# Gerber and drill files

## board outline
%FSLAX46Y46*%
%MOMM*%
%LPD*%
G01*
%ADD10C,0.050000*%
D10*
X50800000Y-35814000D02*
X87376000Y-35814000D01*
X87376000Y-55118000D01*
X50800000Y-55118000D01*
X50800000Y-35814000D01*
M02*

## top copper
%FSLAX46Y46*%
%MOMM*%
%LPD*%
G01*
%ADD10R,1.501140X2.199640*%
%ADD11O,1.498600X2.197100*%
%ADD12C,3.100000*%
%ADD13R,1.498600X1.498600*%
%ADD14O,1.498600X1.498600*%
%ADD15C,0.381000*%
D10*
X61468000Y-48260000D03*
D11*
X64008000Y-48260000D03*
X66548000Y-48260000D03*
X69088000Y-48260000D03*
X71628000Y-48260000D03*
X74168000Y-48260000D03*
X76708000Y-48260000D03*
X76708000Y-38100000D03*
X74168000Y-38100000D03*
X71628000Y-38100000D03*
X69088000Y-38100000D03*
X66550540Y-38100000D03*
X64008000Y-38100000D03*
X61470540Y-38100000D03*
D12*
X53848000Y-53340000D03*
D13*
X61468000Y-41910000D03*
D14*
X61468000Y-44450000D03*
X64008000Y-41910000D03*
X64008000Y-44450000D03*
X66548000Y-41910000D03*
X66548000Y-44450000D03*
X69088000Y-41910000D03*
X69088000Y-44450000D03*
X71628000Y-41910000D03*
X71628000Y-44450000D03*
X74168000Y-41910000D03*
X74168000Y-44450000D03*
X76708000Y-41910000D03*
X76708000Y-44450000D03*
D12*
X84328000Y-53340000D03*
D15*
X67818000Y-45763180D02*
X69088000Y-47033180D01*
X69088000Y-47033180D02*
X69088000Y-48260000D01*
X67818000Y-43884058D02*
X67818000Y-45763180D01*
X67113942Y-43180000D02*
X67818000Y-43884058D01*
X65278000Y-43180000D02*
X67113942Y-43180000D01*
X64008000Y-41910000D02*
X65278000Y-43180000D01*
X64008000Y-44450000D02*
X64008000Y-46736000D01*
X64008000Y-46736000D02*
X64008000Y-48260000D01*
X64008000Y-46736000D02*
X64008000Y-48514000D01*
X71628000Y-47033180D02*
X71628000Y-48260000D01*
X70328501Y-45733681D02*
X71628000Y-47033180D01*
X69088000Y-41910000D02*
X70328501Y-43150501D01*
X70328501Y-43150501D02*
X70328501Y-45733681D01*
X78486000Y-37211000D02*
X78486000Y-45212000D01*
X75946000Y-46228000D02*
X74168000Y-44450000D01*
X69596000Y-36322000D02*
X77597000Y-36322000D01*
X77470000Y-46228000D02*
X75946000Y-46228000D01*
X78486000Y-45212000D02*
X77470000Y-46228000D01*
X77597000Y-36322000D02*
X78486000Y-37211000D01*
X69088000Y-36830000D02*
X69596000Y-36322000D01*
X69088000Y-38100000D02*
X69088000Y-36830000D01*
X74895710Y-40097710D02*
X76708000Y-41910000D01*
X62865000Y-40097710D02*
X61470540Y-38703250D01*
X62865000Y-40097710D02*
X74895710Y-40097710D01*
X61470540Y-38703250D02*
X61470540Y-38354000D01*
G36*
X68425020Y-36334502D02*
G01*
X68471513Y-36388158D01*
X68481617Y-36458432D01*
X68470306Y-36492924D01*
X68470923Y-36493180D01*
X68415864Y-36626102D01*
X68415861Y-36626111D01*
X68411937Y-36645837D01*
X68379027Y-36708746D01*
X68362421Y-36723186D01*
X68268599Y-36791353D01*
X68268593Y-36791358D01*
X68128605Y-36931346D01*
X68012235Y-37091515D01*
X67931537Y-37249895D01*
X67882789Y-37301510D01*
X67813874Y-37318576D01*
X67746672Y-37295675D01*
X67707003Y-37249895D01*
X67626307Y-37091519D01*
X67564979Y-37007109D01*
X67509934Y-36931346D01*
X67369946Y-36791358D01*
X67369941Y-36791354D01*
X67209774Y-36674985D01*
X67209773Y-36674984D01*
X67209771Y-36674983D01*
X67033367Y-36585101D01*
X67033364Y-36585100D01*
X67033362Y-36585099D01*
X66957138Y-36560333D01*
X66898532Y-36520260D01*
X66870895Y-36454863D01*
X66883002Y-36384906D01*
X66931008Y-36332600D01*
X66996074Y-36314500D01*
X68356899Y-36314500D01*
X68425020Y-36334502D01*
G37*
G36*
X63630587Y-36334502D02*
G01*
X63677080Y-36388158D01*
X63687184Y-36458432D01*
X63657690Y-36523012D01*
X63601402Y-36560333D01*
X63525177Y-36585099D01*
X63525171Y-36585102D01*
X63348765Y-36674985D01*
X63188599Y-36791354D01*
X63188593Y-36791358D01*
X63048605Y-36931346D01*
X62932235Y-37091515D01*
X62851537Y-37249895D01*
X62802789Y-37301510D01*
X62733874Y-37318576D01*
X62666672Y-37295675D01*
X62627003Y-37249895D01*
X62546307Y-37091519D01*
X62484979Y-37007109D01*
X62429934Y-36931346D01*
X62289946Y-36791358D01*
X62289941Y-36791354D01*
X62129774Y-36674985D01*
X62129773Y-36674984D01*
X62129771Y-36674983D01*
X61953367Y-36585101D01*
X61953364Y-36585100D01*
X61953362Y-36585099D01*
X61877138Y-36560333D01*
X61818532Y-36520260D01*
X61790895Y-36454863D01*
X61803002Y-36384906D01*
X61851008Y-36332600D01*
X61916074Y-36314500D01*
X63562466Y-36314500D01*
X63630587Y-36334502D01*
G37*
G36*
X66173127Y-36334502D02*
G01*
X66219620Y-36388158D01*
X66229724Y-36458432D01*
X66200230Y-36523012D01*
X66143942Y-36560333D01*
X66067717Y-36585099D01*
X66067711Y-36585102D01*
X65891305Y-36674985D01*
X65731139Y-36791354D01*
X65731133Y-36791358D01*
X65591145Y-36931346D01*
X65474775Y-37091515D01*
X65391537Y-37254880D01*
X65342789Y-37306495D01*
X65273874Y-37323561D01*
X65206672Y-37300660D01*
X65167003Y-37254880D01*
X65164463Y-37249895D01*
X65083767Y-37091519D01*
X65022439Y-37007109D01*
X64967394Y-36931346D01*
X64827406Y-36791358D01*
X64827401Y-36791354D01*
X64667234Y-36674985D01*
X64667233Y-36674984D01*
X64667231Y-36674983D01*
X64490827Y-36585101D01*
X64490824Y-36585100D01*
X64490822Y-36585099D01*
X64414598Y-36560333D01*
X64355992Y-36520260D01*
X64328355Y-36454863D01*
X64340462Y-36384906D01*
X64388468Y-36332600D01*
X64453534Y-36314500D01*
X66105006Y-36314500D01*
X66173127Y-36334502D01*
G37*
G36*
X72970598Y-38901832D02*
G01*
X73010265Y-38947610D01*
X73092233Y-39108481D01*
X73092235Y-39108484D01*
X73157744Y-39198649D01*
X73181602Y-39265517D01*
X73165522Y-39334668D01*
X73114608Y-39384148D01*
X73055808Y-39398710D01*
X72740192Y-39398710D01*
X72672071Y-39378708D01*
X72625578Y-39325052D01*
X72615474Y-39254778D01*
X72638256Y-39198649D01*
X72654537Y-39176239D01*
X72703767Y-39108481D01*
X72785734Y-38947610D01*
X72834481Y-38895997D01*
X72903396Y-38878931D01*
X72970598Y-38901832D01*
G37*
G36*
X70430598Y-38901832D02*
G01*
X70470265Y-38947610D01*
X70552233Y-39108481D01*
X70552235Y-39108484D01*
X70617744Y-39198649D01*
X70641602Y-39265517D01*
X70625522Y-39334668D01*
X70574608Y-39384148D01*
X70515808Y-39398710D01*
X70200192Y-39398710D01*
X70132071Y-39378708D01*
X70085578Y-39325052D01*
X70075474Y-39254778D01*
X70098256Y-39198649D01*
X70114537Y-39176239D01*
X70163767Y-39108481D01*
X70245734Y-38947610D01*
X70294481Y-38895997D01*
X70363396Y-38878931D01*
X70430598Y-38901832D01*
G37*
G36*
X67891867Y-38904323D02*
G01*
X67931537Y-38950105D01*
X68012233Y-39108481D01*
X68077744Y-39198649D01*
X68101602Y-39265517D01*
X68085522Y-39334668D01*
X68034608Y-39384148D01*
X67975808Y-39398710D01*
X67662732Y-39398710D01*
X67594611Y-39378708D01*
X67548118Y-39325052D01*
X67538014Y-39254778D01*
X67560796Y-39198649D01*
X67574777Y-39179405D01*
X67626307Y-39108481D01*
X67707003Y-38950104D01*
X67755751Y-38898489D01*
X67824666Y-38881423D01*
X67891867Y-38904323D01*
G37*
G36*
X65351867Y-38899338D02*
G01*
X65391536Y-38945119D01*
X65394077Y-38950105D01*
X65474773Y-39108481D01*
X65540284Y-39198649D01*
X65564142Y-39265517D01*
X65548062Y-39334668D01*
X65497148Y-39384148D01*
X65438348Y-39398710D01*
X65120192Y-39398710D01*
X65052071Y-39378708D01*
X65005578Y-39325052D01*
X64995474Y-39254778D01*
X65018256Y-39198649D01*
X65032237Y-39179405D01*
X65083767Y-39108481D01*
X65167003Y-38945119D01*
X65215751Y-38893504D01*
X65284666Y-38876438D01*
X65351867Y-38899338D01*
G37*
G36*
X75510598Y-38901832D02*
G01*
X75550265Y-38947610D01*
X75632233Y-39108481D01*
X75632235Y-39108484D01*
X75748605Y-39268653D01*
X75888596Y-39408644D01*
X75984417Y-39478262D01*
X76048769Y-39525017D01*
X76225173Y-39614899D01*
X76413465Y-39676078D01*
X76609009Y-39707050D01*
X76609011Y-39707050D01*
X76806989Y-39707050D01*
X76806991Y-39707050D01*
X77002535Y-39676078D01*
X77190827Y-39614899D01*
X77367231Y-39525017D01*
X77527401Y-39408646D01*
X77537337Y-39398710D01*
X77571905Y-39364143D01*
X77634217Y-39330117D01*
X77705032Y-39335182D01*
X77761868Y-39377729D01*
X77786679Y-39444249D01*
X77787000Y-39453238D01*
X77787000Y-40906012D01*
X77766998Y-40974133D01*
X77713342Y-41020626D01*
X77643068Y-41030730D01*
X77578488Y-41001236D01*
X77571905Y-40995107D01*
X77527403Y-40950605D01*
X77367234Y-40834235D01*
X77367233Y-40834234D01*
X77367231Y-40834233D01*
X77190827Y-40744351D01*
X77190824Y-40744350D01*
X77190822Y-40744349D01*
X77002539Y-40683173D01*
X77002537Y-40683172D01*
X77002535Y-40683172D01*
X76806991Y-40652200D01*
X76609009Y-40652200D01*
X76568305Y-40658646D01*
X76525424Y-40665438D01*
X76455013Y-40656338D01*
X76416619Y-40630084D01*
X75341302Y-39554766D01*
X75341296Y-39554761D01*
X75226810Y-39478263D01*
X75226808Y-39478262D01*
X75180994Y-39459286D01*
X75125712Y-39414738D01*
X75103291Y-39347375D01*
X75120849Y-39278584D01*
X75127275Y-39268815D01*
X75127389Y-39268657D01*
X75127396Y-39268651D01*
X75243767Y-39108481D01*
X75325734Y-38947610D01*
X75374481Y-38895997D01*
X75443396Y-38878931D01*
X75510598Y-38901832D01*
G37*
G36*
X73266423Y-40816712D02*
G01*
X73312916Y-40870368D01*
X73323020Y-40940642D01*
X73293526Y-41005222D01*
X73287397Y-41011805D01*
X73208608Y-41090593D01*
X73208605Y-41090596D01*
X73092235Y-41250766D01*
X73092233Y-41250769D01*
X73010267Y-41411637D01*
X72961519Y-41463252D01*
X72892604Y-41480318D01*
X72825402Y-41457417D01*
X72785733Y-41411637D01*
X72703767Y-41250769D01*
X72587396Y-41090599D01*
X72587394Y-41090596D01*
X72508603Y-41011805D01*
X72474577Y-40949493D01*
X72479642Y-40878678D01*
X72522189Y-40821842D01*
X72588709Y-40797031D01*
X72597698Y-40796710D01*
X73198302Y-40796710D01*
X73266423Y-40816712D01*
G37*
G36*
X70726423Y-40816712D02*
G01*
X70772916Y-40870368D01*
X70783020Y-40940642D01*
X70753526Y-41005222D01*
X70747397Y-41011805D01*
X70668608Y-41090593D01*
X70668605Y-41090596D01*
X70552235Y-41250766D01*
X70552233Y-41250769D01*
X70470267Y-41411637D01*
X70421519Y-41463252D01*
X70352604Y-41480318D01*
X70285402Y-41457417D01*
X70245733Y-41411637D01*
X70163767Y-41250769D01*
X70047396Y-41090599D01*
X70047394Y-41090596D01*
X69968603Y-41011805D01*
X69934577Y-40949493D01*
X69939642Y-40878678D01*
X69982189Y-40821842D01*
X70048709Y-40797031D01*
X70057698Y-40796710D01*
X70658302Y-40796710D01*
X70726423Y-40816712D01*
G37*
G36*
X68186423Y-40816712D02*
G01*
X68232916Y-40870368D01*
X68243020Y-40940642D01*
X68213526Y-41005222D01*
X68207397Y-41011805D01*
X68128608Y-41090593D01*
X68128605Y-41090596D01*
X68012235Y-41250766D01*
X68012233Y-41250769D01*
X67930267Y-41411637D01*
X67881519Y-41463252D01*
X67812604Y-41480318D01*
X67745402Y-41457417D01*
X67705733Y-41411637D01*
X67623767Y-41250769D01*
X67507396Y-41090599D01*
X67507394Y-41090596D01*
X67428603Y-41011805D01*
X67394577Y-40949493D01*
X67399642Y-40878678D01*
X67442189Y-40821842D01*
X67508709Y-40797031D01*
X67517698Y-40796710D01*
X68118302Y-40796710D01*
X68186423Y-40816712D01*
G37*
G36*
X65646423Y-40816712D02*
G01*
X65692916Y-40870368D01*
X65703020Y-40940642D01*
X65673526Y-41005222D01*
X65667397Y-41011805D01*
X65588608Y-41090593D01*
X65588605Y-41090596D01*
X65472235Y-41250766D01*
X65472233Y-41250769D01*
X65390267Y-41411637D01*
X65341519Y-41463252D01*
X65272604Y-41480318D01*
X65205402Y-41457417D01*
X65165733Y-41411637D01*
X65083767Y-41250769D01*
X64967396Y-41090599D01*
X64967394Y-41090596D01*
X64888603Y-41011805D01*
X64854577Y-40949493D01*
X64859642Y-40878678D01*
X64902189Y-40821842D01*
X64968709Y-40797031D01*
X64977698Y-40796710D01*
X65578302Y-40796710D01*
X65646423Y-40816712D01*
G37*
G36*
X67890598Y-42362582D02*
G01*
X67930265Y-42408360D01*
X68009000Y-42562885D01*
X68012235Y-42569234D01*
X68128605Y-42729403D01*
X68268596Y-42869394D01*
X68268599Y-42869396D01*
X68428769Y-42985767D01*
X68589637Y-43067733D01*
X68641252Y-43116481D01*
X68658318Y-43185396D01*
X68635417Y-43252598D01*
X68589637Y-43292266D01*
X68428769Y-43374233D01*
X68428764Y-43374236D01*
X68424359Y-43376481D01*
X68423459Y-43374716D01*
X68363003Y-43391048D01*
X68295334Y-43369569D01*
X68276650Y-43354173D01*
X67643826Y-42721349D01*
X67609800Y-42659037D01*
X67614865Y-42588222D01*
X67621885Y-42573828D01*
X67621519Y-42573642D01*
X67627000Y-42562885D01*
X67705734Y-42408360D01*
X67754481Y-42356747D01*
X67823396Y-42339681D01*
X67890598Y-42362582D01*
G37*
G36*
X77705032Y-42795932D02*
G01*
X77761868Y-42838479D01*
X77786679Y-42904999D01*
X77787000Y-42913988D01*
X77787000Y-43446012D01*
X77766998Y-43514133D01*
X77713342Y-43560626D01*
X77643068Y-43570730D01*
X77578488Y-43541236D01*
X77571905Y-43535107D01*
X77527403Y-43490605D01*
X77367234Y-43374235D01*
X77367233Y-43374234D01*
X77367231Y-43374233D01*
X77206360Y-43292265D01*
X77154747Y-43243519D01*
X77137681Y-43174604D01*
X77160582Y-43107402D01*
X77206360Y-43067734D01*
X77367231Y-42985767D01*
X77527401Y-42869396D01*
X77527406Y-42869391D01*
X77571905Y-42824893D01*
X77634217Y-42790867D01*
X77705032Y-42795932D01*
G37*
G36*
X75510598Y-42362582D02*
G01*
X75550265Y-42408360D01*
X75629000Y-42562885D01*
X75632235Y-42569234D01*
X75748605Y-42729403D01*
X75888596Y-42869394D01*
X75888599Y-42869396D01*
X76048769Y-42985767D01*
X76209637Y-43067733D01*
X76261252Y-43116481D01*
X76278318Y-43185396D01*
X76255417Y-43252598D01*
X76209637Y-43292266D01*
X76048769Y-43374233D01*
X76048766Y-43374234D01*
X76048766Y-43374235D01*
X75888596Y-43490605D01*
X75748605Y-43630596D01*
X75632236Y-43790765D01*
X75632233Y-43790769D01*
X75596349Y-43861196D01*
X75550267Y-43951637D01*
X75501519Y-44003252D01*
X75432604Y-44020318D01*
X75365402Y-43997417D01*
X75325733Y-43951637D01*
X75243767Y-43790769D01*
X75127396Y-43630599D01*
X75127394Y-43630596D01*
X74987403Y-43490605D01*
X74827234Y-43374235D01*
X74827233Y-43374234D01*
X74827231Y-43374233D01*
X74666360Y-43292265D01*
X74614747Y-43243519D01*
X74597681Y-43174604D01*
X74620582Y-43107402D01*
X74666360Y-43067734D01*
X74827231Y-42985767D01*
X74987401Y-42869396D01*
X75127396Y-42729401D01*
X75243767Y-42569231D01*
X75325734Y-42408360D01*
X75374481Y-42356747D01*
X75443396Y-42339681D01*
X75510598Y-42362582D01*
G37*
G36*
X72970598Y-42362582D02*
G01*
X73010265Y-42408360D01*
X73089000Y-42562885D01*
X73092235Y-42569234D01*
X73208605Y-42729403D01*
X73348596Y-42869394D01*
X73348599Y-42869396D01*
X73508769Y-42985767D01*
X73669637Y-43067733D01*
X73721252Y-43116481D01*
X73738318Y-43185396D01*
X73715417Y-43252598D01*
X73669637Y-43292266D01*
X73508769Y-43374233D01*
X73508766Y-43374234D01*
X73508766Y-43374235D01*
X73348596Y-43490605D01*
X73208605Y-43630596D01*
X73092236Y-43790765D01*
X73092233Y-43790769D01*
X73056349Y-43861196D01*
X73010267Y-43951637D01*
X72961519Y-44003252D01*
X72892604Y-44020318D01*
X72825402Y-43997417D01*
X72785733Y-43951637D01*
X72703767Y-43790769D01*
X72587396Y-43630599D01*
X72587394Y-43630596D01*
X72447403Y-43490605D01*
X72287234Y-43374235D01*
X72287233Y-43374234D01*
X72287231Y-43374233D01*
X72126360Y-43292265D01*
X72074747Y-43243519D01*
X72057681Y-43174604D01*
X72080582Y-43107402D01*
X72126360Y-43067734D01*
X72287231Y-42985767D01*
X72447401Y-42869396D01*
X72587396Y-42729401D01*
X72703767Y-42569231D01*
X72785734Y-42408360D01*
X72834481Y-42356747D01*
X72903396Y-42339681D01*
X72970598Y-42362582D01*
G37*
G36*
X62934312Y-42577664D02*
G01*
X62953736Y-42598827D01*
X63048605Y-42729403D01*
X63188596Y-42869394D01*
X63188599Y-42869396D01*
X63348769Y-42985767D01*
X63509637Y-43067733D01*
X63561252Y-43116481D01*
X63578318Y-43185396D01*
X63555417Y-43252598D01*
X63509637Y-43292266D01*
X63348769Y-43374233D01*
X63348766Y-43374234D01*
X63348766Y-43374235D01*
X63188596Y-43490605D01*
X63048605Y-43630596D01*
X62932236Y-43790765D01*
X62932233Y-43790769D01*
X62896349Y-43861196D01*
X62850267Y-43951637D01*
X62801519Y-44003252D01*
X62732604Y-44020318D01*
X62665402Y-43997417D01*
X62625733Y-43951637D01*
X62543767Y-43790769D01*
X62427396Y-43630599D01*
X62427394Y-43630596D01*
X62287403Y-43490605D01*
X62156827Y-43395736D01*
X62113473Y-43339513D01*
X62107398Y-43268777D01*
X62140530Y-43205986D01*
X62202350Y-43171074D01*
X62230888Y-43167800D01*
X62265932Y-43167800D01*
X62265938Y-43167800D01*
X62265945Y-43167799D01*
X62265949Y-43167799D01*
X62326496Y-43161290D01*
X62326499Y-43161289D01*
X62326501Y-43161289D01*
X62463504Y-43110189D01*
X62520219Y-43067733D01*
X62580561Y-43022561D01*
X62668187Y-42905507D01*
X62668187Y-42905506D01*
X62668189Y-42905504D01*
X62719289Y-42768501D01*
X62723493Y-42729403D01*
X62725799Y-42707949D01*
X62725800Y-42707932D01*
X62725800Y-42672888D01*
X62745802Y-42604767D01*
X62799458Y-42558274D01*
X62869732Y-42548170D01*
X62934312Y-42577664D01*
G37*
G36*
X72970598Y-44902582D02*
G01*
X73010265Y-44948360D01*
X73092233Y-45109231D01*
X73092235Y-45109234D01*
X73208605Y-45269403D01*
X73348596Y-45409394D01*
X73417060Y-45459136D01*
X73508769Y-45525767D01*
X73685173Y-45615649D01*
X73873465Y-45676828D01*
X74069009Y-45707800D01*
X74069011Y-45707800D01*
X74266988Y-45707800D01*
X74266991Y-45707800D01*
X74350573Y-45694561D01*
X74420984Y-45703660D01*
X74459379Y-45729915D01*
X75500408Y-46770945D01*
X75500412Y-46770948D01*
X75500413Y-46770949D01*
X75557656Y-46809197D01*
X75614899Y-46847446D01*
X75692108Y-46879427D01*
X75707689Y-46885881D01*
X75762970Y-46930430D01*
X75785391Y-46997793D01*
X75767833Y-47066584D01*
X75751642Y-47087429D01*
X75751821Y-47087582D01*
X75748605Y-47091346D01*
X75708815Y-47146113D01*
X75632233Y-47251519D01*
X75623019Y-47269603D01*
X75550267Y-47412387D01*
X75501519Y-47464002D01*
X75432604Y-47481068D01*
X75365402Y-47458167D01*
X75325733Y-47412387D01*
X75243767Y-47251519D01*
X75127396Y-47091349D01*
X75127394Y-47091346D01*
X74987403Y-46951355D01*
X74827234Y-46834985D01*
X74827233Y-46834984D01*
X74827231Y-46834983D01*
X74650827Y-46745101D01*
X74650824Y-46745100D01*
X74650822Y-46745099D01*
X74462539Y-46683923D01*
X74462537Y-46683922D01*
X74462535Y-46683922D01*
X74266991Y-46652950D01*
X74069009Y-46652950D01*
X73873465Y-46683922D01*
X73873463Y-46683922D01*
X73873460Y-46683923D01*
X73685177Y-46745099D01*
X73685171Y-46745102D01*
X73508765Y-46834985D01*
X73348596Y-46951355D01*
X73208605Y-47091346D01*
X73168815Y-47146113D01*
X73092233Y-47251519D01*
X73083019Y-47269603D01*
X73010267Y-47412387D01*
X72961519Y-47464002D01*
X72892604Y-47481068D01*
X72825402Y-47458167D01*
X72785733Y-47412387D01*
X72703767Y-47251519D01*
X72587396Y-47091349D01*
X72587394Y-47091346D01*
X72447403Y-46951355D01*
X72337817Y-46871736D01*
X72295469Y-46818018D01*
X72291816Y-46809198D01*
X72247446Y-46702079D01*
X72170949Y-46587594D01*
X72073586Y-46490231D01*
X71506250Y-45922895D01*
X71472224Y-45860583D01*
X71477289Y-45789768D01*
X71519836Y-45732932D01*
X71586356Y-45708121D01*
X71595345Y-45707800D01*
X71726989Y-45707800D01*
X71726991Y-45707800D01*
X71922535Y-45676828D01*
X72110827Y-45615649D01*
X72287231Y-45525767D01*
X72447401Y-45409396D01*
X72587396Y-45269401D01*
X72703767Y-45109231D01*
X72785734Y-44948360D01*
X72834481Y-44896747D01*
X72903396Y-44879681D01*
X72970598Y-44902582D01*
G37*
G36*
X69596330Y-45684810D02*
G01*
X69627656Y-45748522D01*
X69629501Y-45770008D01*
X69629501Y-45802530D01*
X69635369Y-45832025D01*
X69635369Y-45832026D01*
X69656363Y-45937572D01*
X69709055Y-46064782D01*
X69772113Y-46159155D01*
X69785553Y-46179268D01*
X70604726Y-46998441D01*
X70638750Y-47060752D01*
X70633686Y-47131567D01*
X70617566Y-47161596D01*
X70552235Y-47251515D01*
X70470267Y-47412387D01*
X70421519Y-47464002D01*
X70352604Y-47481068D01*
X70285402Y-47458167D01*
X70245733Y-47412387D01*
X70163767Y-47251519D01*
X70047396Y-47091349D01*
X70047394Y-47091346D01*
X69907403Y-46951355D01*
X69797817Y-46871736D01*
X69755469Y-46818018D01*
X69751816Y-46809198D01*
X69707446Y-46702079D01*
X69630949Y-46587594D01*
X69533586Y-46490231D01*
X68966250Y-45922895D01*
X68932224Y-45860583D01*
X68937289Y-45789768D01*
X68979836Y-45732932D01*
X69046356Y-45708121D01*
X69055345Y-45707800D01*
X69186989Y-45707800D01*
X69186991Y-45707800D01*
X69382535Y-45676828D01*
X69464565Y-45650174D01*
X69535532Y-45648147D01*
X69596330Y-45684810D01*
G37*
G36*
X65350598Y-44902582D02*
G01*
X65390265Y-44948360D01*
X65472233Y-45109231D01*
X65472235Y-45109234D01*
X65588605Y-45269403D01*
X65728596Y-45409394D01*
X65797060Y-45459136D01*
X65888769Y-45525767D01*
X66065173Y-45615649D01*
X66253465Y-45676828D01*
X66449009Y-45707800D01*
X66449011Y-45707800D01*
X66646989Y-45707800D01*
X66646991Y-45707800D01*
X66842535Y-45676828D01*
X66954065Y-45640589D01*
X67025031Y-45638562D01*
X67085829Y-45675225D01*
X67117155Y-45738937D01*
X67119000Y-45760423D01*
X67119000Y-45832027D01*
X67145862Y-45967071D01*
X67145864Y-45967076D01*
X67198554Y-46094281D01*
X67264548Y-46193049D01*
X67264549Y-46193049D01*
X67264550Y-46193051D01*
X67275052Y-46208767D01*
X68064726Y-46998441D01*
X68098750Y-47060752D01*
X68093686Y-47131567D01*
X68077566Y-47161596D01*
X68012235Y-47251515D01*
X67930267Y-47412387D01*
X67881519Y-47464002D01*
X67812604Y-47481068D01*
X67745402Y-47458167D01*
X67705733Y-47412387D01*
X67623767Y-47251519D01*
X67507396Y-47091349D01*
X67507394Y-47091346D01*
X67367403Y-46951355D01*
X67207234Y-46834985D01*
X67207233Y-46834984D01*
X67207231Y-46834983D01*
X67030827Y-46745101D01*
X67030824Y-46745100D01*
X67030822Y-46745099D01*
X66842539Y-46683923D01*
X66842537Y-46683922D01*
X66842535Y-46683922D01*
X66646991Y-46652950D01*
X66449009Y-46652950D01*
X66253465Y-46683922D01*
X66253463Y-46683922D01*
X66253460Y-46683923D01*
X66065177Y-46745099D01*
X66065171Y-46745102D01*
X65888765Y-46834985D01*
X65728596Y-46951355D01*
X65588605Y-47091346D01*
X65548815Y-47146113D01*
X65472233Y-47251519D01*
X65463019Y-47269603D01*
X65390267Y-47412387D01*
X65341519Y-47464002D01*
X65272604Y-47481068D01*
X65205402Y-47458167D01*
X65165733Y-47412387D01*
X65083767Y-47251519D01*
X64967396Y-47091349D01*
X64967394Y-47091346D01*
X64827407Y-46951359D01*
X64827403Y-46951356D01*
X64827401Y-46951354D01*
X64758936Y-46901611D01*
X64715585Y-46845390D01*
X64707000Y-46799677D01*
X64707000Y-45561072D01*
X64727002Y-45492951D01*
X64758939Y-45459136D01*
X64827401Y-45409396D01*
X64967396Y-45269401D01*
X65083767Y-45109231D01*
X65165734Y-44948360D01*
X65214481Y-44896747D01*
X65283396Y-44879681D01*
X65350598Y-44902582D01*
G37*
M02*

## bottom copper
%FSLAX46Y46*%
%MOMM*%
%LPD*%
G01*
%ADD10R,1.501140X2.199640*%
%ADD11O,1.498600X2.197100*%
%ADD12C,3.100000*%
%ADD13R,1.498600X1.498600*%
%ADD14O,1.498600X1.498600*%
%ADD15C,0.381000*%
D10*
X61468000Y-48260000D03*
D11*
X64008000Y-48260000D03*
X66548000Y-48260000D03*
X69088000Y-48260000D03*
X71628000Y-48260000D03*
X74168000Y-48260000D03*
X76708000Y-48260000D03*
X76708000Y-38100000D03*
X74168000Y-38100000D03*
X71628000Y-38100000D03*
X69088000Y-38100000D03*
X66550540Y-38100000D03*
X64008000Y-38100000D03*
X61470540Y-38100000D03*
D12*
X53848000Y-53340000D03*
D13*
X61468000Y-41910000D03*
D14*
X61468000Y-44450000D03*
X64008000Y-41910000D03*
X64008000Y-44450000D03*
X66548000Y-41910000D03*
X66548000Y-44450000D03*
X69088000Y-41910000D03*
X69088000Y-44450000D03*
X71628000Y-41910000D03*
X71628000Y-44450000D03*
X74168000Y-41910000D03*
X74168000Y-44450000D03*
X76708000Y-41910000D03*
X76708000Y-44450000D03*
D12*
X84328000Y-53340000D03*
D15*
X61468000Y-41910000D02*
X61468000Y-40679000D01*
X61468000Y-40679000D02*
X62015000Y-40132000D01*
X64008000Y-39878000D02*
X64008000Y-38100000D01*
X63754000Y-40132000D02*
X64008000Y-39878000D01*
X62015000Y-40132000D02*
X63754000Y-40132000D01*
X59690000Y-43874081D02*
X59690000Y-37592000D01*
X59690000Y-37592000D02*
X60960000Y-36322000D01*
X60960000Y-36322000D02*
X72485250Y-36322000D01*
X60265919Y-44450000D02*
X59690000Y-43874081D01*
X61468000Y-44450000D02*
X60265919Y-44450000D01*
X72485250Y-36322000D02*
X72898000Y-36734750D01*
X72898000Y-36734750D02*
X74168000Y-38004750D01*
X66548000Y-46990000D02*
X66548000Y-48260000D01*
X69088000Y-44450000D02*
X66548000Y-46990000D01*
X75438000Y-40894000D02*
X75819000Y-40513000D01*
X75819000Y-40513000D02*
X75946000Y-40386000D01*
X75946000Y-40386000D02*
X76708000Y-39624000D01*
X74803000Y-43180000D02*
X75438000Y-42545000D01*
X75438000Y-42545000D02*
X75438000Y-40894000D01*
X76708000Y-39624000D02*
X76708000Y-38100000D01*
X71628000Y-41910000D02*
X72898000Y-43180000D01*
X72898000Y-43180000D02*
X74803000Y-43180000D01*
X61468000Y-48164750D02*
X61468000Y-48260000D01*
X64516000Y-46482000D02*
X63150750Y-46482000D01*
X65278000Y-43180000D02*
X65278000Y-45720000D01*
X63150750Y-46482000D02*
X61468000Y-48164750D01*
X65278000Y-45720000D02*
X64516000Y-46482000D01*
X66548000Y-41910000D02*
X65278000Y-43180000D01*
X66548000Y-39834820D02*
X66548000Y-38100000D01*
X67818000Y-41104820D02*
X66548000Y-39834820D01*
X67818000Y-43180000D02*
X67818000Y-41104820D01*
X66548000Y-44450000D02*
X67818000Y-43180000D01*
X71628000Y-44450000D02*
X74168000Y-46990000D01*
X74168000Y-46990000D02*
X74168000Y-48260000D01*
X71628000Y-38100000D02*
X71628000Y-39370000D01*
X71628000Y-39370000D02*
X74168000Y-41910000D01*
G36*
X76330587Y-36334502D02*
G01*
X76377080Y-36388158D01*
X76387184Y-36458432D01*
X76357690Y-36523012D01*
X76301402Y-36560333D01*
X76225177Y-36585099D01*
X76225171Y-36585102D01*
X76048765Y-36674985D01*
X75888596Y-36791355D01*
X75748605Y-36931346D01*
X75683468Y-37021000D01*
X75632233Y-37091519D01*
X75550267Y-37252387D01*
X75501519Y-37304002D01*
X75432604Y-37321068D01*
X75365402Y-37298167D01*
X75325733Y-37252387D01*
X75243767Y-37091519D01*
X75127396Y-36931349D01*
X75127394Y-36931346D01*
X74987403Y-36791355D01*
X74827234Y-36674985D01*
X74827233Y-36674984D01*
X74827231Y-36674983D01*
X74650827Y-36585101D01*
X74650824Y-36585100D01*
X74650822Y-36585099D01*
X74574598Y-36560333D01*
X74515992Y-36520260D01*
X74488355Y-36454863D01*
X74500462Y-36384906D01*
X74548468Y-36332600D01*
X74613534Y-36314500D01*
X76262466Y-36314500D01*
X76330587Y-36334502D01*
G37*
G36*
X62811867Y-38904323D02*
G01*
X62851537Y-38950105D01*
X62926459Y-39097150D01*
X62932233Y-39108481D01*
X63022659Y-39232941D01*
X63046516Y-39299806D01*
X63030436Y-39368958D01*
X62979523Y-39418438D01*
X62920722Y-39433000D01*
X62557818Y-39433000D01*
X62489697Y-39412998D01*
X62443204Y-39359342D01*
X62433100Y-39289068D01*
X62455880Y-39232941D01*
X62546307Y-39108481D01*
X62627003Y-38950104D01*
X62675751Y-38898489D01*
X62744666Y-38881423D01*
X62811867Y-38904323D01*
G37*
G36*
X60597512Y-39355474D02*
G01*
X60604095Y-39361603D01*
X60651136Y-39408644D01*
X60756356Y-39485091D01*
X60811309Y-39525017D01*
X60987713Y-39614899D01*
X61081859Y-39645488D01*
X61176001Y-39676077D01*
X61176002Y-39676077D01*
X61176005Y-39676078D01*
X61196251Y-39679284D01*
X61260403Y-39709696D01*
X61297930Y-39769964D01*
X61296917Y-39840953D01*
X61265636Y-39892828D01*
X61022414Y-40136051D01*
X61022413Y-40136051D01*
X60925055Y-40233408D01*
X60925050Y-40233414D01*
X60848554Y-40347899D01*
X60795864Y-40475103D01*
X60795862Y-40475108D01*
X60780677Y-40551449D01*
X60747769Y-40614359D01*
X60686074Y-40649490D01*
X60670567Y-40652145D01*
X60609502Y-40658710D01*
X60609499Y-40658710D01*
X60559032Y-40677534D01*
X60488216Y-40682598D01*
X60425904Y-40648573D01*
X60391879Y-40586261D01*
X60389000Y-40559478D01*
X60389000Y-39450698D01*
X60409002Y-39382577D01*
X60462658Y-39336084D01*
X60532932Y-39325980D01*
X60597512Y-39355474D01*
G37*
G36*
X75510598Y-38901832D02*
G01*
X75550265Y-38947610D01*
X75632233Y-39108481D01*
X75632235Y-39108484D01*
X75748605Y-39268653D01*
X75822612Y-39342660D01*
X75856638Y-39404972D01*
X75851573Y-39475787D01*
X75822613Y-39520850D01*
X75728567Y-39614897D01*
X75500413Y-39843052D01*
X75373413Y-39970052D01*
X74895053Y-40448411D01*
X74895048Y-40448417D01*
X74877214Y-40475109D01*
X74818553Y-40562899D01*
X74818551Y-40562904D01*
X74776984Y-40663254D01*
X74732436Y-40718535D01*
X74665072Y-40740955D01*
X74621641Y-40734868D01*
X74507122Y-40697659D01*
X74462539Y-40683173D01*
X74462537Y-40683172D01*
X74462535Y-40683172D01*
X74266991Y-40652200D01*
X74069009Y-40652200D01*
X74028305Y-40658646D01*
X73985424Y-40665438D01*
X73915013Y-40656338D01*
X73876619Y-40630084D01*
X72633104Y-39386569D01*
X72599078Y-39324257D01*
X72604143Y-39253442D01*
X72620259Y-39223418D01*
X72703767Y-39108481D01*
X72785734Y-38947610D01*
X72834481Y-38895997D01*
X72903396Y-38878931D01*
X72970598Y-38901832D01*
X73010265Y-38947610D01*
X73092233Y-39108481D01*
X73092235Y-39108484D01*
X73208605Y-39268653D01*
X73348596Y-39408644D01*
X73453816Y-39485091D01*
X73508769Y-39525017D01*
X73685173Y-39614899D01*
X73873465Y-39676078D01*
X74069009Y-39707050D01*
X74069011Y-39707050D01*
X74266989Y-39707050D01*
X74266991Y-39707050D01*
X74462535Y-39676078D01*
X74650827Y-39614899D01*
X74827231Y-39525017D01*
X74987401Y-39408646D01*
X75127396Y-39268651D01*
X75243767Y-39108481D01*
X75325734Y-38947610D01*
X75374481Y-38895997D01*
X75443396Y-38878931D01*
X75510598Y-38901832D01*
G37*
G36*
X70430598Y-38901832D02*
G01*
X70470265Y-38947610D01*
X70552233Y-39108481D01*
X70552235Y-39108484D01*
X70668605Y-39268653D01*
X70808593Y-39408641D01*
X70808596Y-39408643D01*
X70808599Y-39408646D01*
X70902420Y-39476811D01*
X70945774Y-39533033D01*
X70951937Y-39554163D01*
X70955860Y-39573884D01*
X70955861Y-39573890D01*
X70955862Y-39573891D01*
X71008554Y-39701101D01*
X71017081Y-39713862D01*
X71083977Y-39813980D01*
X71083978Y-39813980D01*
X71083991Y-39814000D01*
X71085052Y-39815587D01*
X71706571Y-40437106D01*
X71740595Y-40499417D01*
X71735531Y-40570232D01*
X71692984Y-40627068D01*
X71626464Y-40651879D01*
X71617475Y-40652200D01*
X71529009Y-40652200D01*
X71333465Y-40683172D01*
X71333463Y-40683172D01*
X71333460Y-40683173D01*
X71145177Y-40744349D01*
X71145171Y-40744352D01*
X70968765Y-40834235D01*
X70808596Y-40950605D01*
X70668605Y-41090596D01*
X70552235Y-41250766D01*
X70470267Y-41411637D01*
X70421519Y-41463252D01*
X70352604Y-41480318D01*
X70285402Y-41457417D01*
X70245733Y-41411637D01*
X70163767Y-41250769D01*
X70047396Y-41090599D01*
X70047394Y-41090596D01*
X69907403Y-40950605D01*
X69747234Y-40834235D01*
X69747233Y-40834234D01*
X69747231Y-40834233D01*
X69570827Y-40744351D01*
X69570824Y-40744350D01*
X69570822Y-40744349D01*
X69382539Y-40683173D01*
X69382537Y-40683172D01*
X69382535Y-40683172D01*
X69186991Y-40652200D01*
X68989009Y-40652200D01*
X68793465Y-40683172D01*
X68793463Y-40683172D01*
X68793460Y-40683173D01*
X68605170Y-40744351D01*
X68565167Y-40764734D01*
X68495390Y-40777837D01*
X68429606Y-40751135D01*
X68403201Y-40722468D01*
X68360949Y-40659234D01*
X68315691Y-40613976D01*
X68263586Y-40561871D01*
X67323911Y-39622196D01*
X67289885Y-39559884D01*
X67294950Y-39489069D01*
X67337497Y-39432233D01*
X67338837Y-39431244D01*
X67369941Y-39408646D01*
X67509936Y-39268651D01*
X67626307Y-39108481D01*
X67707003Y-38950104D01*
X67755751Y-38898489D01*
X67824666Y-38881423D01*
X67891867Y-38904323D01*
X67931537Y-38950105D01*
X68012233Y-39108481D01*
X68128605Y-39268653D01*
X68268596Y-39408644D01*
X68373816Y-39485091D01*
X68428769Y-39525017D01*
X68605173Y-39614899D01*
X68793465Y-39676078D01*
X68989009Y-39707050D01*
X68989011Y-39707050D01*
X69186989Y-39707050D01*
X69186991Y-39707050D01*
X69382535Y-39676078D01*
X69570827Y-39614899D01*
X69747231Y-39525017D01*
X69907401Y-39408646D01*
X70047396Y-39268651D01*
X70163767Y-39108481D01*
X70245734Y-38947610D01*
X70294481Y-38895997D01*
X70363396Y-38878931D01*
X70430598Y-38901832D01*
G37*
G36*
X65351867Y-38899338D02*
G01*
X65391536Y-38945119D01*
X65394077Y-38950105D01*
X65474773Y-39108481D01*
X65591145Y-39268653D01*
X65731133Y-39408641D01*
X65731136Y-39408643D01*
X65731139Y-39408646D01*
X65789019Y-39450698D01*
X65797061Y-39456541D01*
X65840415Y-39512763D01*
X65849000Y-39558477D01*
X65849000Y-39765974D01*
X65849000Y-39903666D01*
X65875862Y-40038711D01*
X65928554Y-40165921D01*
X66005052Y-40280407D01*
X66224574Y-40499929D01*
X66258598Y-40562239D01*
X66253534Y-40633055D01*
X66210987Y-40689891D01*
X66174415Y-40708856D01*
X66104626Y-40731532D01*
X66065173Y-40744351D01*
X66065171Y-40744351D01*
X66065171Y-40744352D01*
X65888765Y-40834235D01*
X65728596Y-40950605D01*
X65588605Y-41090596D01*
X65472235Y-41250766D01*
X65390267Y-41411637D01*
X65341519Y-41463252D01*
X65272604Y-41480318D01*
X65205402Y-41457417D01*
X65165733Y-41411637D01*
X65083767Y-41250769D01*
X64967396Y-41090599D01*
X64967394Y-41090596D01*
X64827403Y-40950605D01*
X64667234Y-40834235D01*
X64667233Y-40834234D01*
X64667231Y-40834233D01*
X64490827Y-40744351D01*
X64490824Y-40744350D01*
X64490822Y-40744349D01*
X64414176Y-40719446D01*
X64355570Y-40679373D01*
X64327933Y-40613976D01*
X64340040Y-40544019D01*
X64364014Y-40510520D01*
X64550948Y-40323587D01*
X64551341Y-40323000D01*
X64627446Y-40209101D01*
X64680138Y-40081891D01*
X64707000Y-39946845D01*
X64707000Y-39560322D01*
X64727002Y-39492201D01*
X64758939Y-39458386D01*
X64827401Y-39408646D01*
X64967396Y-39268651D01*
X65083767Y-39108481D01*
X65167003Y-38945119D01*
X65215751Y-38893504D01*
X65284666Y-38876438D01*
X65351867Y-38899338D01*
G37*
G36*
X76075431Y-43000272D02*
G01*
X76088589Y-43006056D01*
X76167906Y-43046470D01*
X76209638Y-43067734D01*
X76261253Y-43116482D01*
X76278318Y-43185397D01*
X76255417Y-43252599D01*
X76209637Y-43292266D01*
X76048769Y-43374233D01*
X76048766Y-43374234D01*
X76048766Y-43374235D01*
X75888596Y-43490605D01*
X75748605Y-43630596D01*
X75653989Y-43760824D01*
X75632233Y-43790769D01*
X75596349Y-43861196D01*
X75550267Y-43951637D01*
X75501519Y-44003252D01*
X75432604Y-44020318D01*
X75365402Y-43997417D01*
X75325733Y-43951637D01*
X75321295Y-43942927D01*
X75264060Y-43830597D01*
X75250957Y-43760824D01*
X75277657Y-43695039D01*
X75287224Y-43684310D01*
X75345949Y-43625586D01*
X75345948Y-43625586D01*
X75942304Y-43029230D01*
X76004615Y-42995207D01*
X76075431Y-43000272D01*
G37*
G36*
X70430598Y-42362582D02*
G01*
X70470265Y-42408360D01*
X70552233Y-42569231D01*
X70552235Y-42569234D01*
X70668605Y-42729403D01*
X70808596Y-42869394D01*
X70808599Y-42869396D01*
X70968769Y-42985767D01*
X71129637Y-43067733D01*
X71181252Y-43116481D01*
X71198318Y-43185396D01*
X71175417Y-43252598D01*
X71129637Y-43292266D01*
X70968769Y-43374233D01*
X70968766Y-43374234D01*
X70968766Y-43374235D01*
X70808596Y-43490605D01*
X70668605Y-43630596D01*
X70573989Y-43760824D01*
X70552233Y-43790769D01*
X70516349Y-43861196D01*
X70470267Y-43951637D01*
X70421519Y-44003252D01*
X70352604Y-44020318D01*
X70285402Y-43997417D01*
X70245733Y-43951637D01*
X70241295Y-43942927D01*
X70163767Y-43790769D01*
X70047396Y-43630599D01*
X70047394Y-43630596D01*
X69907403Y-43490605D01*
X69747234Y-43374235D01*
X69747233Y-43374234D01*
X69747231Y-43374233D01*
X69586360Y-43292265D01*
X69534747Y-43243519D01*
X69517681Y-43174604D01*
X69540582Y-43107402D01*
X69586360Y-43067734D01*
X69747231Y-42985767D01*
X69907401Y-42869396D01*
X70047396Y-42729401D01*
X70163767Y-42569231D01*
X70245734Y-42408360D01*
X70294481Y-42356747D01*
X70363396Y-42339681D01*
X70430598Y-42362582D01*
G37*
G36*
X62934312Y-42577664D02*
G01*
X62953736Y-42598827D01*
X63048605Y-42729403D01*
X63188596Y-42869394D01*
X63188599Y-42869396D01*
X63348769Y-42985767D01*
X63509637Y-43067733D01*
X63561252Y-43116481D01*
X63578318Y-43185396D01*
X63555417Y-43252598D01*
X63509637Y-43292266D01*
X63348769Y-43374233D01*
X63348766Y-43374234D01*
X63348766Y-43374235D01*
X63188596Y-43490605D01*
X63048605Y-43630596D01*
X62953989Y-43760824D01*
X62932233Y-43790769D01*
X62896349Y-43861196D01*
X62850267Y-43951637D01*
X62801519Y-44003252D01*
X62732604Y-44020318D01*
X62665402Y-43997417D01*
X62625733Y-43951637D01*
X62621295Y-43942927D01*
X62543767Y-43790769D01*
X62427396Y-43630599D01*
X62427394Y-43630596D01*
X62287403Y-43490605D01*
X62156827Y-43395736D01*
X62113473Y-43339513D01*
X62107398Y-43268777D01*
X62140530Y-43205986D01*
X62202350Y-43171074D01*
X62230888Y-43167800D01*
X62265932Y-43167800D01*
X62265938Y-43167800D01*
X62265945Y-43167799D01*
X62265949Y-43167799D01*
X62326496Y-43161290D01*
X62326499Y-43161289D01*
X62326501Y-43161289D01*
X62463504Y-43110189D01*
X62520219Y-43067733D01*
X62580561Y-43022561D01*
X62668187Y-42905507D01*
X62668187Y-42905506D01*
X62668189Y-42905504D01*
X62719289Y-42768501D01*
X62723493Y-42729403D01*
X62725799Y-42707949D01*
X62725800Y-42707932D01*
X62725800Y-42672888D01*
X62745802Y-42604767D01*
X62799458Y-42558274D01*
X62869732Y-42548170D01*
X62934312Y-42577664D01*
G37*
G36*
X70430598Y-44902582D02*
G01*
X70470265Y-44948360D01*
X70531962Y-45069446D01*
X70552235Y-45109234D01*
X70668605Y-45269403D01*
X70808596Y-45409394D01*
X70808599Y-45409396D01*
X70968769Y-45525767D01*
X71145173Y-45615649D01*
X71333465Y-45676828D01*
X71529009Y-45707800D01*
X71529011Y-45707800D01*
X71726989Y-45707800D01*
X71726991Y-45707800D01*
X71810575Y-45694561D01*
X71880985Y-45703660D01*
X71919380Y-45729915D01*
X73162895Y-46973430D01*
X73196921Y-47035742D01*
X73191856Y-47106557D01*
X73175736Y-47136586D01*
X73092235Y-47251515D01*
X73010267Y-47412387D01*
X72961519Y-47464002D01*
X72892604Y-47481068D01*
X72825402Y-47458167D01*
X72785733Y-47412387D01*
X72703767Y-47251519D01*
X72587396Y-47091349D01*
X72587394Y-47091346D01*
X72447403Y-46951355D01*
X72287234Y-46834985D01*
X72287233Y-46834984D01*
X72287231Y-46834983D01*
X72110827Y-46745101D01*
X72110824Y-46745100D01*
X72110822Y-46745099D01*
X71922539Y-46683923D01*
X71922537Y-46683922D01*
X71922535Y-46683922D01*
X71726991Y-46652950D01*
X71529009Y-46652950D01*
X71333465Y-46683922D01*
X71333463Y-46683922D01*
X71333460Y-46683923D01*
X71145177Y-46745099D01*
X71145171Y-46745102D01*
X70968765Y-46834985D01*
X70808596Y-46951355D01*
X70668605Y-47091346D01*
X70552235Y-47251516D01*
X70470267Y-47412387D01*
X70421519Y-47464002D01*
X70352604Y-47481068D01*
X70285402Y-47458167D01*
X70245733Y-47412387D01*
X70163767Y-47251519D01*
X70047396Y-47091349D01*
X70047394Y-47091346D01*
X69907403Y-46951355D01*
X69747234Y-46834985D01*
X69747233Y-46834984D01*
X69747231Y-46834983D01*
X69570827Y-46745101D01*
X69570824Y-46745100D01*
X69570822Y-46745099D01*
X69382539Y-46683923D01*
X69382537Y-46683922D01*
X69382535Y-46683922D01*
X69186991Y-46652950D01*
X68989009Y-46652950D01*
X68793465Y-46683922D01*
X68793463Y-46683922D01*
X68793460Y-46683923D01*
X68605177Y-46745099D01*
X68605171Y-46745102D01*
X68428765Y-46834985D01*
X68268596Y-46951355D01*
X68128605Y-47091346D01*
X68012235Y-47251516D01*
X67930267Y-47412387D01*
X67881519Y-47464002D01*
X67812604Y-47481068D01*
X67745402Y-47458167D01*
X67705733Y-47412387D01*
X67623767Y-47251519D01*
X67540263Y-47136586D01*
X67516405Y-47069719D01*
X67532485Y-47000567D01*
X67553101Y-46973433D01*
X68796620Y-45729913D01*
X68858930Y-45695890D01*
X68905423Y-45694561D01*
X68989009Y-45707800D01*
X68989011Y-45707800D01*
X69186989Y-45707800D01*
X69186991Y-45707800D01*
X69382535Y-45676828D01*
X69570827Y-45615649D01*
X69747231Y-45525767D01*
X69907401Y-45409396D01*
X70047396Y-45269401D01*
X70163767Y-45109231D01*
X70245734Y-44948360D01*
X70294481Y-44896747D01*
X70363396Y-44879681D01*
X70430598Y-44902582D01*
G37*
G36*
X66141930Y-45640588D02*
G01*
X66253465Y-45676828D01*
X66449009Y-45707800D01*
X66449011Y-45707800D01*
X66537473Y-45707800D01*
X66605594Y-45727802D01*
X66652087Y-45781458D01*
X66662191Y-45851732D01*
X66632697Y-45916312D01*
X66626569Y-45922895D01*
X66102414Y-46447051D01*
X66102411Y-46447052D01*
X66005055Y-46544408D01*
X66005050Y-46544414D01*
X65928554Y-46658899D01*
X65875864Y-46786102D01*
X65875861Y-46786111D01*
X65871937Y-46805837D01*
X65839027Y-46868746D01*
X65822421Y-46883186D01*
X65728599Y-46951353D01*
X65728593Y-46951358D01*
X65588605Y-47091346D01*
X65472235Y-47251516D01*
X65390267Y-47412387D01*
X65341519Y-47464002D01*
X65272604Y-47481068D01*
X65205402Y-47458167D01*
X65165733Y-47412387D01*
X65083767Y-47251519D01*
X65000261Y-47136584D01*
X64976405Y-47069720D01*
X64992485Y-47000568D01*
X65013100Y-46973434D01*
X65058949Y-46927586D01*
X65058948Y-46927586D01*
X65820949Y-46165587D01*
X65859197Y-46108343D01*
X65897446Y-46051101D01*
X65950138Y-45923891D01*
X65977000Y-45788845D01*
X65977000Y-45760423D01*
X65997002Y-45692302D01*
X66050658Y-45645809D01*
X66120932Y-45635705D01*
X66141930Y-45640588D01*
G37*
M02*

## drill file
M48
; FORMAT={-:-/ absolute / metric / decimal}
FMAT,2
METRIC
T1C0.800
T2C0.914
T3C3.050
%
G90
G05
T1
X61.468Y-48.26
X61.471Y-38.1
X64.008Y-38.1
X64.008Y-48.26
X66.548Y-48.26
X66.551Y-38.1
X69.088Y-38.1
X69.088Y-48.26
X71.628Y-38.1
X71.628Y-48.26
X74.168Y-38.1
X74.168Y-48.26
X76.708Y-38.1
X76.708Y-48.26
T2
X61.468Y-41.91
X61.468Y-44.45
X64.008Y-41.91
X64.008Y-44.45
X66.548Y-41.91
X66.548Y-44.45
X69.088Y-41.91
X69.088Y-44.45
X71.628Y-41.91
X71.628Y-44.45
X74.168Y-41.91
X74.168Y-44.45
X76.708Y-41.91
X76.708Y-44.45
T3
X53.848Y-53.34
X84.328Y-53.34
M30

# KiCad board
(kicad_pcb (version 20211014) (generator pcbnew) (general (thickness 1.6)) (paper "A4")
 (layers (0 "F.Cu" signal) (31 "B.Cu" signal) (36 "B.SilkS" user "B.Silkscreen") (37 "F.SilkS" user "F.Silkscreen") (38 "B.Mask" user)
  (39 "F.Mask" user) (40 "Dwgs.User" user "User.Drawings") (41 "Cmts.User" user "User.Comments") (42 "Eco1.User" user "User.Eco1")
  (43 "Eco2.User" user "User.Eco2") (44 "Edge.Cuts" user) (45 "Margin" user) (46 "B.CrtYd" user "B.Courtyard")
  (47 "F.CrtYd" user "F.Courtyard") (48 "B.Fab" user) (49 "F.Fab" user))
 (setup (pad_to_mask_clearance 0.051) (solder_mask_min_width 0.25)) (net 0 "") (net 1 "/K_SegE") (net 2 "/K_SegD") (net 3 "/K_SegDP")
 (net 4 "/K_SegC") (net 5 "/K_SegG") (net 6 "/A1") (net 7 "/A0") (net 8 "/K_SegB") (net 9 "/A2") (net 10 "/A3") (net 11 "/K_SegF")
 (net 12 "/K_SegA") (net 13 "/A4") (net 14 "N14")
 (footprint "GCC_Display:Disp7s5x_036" (layer "F.Cu") (at 69.088 43.18)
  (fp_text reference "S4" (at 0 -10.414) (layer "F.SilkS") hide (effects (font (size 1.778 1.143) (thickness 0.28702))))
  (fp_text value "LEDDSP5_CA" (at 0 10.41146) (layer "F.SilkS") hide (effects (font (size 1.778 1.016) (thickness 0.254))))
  (pad "1" thru_hole rect locked (at -7.62 5.08 90) (size 2.19964 1.50114) (drill 0.8001) (layers *.Cu *.Mask) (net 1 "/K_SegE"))
  (pad "2" thru_hole oval locked (at -5.08 5.08 90) (size 2.1971 1.4986) (drill 0.8001) (layers *.Cu *.Mask) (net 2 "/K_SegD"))
  (pad "3" thru_hole oval locked (at -2.54 5.08 90) (size 2.1971 1.4986) (drill 0.8001) (layers *.Cu *.Mask) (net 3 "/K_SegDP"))
  (pad "4" thru_hole oval locked (at 0 5.08 90) (size 2.1971 1.4986) (drill 0.8001) (layers *.Cu *.Mask) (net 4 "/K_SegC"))
  (pad "5" thru_hole oval locked (at 2.54 5.08 90) (size 2.1971 1.4986) (drill 0.8001) (layers *.Cu *.Mask) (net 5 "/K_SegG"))
  (pad "6" thru_hole oval locked (at 5.08 5.08 90) (size 2.1971 1.4986) (drill 0.8001) (layers *.Cu *.Mask) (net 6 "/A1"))
  (pad "7" thru_hole oval locked (at 7.62 5.08 90) (size 2.1971 1.4986) (drill 0.8001) (layers *.Cu *.Mask))
  (pad "8" thru_hole oval locked (at 7.62 -5.08 90) (size 2.1971 1.4986) (drill 0.8001) (layers *.Cu *.Mask) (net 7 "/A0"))
  (pad "9" thru_hole oval locked (at 5.08 -5.08 90) (size 2.1971 1.4986) (drill 0.8001) (layers *.Cu *.Mask) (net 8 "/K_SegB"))
  (pad "10" thru_hole oval locked (at 2.54 -5.08 90) (size 2.1971 1.4986) (drill 0.8001) (layers *.Cu *.Mask) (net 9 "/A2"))
  (pad "11" thru_hole oval locked (at 0 -5.08 90) (size 2.1971 1.4986) (drill 0.8001) (layers *.Cu *.Mask) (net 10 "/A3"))
  (pad "12" thru_hole oval locked (at -2.53746 -5.08 90) (size 2.1971 1.4986) (drill 0.8001) (layers *.Cu *.Mask) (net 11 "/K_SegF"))
  (pad "13" thru_hole oval locked (at -5.08 -5.08 90) (size 2.1971 1.4986) (drill 0.8001) (layers *.Cu *.Mask) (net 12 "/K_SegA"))
  (pad "14" thru_hole oval locked (at -7.61746 -5.08 90) (size 2.1971 1.4986) (drill 0.8001) (layers *.Cu *.Mask) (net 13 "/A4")))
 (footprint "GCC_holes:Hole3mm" (layer "B.Cu") (at 53.848 53.34)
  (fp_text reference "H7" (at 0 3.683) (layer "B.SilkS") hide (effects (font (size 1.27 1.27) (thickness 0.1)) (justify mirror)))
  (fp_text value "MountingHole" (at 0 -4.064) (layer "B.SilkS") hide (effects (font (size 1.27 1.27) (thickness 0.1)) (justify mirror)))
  (pad "1" thru_hole circle locked (at 0 0) (size 3.1 3.1) (drill 3.05) (layers *.Cu *.Mask)))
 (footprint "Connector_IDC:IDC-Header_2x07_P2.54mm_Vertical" (layer "B.Cu") (at 61.468 41.91 -90)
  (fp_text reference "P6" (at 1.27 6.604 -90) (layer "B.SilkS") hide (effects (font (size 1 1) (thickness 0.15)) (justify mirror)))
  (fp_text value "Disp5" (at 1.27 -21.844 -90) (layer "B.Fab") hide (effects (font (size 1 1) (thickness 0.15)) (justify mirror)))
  (pad "1" thru_hole rect locked (at 0 0 270) (size 1.4986 1.4986) (drill 0.9144) (layers *.Cu *.Mask) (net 12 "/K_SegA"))
  (pad "2" thru_hole oval locked (at 2.54 0 270) (size 1.4986 1.4986) (drill 0.9144) (layers *.Cu *.Mask) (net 8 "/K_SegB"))
  (pad "3" thru_hole oval locked (at 0 -2.54 270) (size 1.4986 1.4986) (drill 0.9144) (layers *.Cu *.Mask) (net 4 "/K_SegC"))
  (pad "4" thru_hole oval locked (at 2.54 -2.54 270) (size 1.4986 1.4986) (drill 0.9144) (layers *.Cu *.Mask) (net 2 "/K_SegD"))
  (pad "5" thru_hole oval locked (at 0 -5.08 270) (size 1.4986 1.4986) (drill 0.9144) (layers *.Cu *.Mask) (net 1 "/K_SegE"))
  (pad "6" thru_hole oval locked (at 2.54 -5.08 270) (size 1.4986 1.4986) (drill 0.9144) (layers *.Cu *.Mask) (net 11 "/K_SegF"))
  (pad "7" thru_hole oval locked (at 0 -7.62 270) (size 1.4986 1.4986) (drill 0.9144) (layers *.Cu *.Mask) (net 5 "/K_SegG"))
  (pad "8" thru_hole oval locked (at 2.54 -7.62 270) (size 1.4986 1.4986) (drill 0.9144) (layers *.Cu *.Mask) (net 3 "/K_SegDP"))
  (pad "9" thru_hole oval locked (at 0 -10.16 270) (size 1.4986 1.4986) (drill 0.9144) (layers *.Cu *.Mask) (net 7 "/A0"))
  (pad "10" thru_hole oval locked (at 2.54 -10.16 270) (size 1.4986 1.4986) (drill 0.9144) (layers *.Cu *.Mask) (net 6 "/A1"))
  (pad "11" thru_hole oval locked (at 0 -12.7 270) (size 1.4986 1.4986) (drill 0.9144) (layers *.Cu *.Mask) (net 9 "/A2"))
  (pad "12" thru_hole oval locked (at 2.54 -12.7 270) (size 1.4986 1.4986) (drill 0.9144) (layers *.Cu *.Mask) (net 10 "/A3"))
  (pad "13" thru_hole oval locked (at 0 -15.24 270) (size 1.4986 1.4986) (drill 0.9144) (layers *.Cu *.Mask) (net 13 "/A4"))
  (pad "14" thru_hole oval locked (at 2.54 -15.24 270) (size 1.4986 1.4986) (drill 0.9144) (layers *.Cu *.Mask) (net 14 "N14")))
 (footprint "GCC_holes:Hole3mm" (layer "B.Cu") (at 84.328 53.34)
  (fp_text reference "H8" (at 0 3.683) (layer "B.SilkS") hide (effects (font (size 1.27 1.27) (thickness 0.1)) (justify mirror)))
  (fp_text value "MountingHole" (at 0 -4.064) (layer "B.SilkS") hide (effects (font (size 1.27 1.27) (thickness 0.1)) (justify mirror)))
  (pad "1" thru_hole circle locked (at 0 0) (size 3.1 3.1) (drill 3.05) (layers *.Cu *.Mask)))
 (gr_rect (start 50.8 35.814) (end 87.376 55.118) (layer "Edge.Cuts") (width 0.05) (fill none))
 (segment (start 61.468 41.91) (end 61.468 40.679) (width 0.381) (layer "B.Cu") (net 12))
 (segment (start 61.468 40.679) (end 62.015 40.132) (width 0.381) (layer "B.Cu") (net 12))
 (segment (start 64.008 39.878) (end 64.008 38.1) (width 0.381) (layer "B.Cu") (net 12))
 (segment (start 63.754 40.132) (end 64.008 39.878) (width 0.381) (layer "B.Cu") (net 12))
 (segment (start 62.015 40.132) (end 63.754 40.132) (width 0.381) (layer "B.Cu") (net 12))
 (segment (start 59.69 43.874081) (end 59.69 37.592) (width 0.381) (layer "B.Cu") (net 8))
 (segment (start 59.69 37.592) (end 60.96 36.322) (width 0.381) (layer "B.Cu") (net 8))
 (segment (start 60.96 36.322) (end 72.48525 36.322) (width 0.381) (layer "B.Cu") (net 8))
 (segment (start 60.265919 44.45) (end 59.69 43.874081) (width 0.381) (layer "B.Cu") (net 8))
 (segment (start 61.468 44.45) (end 60.265919 44.45) (width 0.381) (layer "B.Cu") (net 8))
 (segment (start 72.48525 36.322) (end 72.898 36.73475) (width 0.381) (layer "B.Cu") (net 8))
 (segment (start 72.898 36.73475) (end 74.168 38.00475) (width 0.381) (layer "B.Cu") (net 8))
 (segment (start 67.818 45.76318) (end 69.088 47.03318) (width 0.381) (layer "F.Cu") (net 4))
 (segment (start 69.088 47.03318) (end 69.088 48.26) (width 0.381) (layer "F.Cu") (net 4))
 (segment (start 67.818 43.884058) (end 67.818 45.76318) (width 0.381) (layer "F.Cu") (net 4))
 (segment (start 67.113942 43.18) (end 67.818 43.884058) (width 0.381) (layer "F.Cu") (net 4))
 (segment (start 65.278 43.18) (end 67.113942 43.18) (width 0.381) (layer "F.Cu") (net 4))
 (segment (start 64.008 41.91) (end 65.278 43.18) (width 0.381) (layer "F.Cu") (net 4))
 (segment (start 66.548 46.99) (end 66.548 48.26) (width 0.381) (layer "B.Cu") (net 3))
 (segment (start 69.088 44.45) (end 66.548 46.99) (width 0.381) (layer "B.Cu") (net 3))
 (segment (start 75.438 40.894) (end 75.819 40.513) (width 0.381) (layer "B.Cu") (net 7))
 (segment (start 75.819 40.513) (end 75.946 40.386) (width 0.381) (layer "B.Cu") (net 7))
 (segment (start 75.946 40.386) (end 76.708 39.624) (width 0.381) (layer "B.Cu") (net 7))
 (segment (start 74.803 43.18) (end 75.438 42.545) (width 0.381) (layer "B.Cu") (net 7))
 (segment (start 75.438 42.545) (end 75.438 40.894) (width 0.381) (layer "B.Cu") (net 7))
 (segment (start 76.708 39.624) (end 76.708 38.1) (width 0.381) (layer "B.Cu") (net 7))
 (segment (start 71.628 41.91) (end 72.898 43.18) (width 0.381) (layer "B.Cu") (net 7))
 (segment (start 72.898 43.18) (end 74.803 43.18) (width 0.381) (layer "B.Cu") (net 7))
 (segment (start 64.008 44.45) (end 64.008 46.736) (width 0.381) (layer "F.Cu") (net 2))
 (segment (start 64.008 46.736) (end 64.008 48.26) (width 0.381) (layer "F.Cu") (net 2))
 (segment (start 64.008 46.736) (end 64.008 48.514) (width 0.381) (layer "F.Cu") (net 2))
 (segment (start 61.468 48.16475) (end 61.468 48.26) (width 0.381) (layer "B.Cu") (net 1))
 (segment (start 64.516 46.482) (end 63.15075 46.482) (width 0.381) (layer "B.Cu") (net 1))
 (segment (start 65.278 43.18) (end 65.278 45.72) (width 0.381) (layer "B.Cu") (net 1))
 (segment (start 63.15075 46.482) (end 61.468 48.16475) (width 0.381) (layer "B.Cu") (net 1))
 (segment (start 65.278 45.72) (end 64.516 46.482) (width 0.381) (layer "B.Cu") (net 1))
 (segment (start 66.548 41.91) (end 65.278 43.18) (width 0.381) (layer "B.Cu") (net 1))
 (segment (start 71.628 47.03318) (end 71.628 48.26) (width 0.381) (layer "F.Cu") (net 5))
 (segment (start 70.328501 45.733681) (end 71.628 47.03318) (width 0.381) (layer "F.Cu") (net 5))
 (segment (start 69.088 41.91) (end 70.328501 43.150501) (width 0.381) (layer "F.Cu") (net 5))
 (segment (start 70.328501 43.150501) (end 70.328501 45.733681) (width 0.381) (layer "F.Cu") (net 5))
 (segment (start 66.548 39.83482) (end 66.548 38.1) (width 0.381) (layer "B.Cu") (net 11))
 (segment (start 67.818 41.10482) (end 66.548 39.83482) (width 0.381) (layer "B.Cu") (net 11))
 (segment (start 67.818 43.18) (end 67.818 41.10482) (width 0.381) (layer "B.Cu") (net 11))
 (segment (start 66.548 44.45) (end 67.818 43.18) (width 0.381) (layer "B.Cu") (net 11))
 (segment (start 71.628 44.45) (end 74.168 46.99) (width 0.381) (layer "B.Cu") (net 6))
 (segment (start 74.168 46.99) (end 74.168 48.26) (width 0.381) (layer "B.Cu") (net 6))
 (segment (start 71.628 38.1) (end 71.628 39.37) (width 0.381) (layer "B.Cu") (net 9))
 (segment (start 71.628 39.37) (end 74.168 41.91) (width 0.381) (layer "B.Cu") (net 9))
 (segment (start 78.486 37.211) (end 78.486 45.212) (width 0.381) (layer "F.Cu") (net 10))
 (segment (start 75.946 46.228) (end 74.168 44.45) (width 0.381) (layer "F.Cu") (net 10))
 (segment (start 69.596 36.322) (end 77.597 36.322) (width 0.381) (layer "F.Cu") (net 10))
 (segment (start 77.47 46.228) (end 75.946 46.228) (width 0.381) (layer "F.Cu") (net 10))
 (segment (start 78.486 45.212) (end 77.47 46.228) (width 0.381) (layer "F.Cu") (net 10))
 (segment (start 77.597 36.322) (end 78.486 37.211) (width 0.381) (layer "F.Cu") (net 10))
 (segment (start 69.088 36.83) (end 69.596 36.322) (width 0.381) (layer "F.Cu") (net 10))
 (segment (start 69.088 38.1) (end 69.088 36.83) (width 0.381) (layer "F.Cu") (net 10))
 (segment (start 74.89571 40.09771) (end 76.708 41.91) (width 0.381) (layer "F.Cu") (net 13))
 (segment (start 62.865 40.09771) (end 61.47054 38.70325) (width 0.381) (layer "F.Cu") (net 13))
 (segment (start 62.865 40.09771) (end 74.89571 40.09771) (width 0.381) (layer "F.Cu") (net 13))
 (segment (start 61.47054 38.70325) (end 61.47054 38.354) (width 0.381) (layer "F.Cu") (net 13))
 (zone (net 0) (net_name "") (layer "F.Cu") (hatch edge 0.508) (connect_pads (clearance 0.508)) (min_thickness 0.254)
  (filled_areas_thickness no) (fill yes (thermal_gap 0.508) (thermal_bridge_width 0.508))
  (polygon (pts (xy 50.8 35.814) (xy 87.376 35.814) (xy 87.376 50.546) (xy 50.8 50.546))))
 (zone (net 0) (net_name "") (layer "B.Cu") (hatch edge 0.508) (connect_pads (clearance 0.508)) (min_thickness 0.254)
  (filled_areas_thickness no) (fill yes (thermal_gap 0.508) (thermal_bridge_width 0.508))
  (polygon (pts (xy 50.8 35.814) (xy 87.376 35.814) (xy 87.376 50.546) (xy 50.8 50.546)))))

